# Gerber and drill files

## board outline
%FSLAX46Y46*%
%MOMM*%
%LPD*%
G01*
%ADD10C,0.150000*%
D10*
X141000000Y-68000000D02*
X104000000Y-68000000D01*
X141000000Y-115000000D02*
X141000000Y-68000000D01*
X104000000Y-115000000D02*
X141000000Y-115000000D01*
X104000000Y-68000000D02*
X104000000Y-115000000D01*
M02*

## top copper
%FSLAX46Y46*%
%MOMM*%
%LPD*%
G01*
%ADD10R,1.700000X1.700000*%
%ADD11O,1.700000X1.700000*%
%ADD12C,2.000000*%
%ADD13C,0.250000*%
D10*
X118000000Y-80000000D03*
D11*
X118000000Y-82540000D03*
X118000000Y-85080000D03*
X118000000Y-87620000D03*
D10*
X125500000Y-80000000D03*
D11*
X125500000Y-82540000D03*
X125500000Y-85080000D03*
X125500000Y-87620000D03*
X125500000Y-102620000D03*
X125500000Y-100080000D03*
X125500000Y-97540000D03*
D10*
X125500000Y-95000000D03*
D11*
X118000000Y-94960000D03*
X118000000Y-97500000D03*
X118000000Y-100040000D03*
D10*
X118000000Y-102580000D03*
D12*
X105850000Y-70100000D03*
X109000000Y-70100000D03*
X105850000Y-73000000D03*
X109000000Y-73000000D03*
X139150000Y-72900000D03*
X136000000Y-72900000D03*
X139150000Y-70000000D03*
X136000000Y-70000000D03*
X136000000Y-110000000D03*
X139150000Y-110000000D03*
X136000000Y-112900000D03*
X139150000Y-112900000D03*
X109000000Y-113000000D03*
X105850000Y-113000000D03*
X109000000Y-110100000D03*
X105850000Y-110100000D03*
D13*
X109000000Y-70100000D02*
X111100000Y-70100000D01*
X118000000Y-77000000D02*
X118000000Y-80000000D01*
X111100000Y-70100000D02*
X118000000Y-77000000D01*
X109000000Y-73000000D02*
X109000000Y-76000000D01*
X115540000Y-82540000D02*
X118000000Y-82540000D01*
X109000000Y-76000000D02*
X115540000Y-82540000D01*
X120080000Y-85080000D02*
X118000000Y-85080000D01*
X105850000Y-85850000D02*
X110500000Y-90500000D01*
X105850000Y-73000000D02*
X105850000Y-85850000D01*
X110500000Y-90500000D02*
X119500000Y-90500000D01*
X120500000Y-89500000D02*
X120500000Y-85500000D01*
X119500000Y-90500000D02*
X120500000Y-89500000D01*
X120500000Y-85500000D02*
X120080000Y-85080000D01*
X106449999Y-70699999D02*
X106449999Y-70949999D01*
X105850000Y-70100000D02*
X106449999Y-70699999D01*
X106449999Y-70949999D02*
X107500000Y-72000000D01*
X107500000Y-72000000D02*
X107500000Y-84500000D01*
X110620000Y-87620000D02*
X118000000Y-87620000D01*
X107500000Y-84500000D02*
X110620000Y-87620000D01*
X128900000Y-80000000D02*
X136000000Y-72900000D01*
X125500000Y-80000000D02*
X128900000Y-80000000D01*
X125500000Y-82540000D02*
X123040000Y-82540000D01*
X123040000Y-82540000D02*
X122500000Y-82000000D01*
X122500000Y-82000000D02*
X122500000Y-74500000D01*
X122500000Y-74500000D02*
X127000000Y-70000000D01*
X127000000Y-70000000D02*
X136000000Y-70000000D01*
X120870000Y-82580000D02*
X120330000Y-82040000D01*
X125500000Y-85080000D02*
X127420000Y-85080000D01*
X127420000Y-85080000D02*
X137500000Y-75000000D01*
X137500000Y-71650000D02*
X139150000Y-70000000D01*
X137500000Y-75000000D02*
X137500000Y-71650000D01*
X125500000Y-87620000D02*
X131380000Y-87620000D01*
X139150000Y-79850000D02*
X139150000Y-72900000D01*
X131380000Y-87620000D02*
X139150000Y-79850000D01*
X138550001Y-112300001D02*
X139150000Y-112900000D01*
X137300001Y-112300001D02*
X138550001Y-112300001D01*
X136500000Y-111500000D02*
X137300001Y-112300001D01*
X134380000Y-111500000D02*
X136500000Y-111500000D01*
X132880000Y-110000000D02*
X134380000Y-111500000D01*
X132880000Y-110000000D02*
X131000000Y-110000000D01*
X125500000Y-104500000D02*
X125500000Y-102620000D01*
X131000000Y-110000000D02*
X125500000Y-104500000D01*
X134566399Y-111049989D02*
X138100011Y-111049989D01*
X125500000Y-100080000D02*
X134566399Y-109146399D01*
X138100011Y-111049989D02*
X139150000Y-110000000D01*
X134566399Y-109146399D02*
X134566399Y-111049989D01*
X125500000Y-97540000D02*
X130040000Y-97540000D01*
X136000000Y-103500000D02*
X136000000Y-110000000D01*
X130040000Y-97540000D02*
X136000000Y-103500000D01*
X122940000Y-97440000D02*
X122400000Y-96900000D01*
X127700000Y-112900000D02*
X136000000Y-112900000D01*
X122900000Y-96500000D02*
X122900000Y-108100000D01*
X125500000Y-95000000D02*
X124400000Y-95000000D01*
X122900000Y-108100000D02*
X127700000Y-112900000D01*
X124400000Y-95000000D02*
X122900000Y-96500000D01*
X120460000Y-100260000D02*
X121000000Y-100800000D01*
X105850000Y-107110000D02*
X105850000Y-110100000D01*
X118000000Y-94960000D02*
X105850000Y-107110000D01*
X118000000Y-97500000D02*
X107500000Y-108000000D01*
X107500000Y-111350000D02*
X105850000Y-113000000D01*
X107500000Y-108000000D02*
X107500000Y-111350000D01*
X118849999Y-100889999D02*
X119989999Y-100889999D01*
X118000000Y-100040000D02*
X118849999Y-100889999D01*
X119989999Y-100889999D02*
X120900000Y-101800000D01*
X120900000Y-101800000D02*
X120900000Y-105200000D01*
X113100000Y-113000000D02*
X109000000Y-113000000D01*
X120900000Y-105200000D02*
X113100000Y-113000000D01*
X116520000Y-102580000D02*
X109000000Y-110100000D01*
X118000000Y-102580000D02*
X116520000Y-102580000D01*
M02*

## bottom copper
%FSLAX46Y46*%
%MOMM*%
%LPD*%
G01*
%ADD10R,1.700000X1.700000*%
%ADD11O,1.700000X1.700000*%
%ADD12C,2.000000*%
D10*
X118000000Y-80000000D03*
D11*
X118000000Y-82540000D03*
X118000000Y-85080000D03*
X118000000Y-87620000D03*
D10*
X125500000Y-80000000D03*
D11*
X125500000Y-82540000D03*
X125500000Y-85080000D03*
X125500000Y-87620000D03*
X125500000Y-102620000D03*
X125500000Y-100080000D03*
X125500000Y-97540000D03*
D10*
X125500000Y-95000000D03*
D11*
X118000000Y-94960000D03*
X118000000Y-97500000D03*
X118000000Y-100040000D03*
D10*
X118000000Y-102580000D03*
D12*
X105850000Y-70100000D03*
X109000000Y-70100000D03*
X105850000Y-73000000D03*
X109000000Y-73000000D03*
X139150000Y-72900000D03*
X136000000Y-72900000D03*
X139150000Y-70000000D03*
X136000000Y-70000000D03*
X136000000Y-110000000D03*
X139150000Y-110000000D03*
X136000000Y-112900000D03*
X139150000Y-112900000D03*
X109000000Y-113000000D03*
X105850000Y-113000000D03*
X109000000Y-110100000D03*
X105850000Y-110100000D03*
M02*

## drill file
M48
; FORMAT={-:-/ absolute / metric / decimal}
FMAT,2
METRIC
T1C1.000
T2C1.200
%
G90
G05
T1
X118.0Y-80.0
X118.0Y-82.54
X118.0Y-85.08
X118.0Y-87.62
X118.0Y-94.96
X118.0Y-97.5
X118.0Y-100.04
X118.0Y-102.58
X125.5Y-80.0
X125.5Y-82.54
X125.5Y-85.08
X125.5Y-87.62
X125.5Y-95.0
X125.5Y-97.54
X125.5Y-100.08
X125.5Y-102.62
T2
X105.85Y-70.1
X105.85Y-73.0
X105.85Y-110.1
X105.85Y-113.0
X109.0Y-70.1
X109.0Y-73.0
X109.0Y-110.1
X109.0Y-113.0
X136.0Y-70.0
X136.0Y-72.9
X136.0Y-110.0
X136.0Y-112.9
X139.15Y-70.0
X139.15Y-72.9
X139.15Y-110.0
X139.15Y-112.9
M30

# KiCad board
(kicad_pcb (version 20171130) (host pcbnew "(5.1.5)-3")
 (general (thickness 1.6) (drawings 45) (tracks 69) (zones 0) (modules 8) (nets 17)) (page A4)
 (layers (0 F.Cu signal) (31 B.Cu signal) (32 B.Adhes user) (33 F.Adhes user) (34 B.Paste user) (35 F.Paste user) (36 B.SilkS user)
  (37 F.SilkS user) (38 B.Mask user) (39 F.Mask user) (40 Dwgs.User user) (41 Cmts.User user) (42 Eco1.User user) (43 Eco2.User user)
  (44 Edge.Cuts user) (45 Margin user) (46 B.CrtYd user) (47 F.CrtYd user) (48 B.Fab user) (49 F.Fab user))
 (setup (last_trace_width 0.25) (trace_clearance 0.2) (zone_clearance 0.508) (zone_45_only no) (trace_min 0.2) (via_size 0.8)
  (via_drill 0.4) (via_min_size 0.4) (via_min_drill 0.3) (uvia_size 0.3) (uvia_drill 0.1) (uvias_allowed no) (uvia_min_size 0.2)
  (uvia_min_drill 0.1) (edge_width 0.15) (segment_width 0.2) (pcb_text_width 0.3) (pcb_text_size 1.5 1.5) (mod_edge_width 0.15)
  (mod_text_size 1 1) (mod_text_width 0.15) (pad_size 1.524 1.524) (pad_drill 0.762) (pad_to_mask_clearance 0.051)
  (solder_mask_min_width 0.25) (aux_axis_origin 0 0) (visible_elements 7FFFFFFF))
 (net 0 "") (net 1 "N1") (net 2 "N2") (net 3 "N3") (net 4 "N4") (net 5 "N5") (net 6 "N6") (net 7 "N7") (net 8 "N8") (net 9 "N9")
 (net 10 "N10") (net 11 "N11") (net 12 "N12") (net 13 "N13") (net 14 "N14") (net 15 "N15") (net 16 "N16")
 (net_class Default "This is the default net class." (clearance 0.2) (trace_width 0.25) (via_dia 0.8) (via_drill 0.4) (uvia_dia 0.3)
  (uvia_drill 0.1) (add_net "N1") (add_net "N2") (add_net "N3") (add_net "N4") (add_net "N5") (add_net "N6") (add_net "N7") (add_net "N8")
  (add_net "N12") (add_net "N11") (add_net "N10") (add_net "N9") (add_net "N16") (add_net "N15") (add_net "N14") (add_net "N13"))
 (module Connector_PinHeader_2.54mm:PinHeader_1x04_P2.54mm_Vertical (layer F.Cu) (at 118 80)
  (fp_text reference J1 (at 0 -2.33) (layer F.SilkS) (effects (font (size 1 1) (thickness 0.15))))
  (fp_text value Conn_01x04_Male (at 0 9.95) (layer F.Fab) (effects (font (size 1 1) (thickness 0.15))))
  (pad 1 thru_hole rect (at 0 0) (size 1.7 1.7) (drill 1) (layers *.Cu *.Mask) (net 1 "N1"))
  (pad 2 thru_hole oval (at 0 2.54) (size 1.7 1.7) (drill 1) (layers *.Cu *.Mask) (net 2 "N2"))
  (pad 3 thru_hole oval (at 0 5.08) (size 1.7 1.7) (drill 1) (layers *.Cu *.Mask) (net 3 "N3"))
  (pad 4 thru_hole oval (at 0 7.62) (size 1.7 1.7) (drill 1) (layers *.Cu *.Mask) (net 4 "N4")))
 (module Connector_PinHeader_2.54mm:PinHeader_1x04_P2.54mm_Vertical (layer F.Cu) (at 125.5 80)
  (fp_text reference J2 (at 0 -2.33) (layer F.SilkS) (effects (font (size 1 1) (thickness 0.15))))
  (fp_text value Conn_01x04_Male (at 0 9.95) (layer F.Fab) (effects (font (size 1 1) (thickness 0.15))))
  (pad 1 thru_hole rect (at 0 0) (size 1.7 1.7) (drill 1) (layers *.Cu *.Mask) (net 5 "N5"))
  (pad 2 thru_hole oval (at 0 2.54) (size 1.7 1.7) (drill 1) (layers *.Cu *.Mask) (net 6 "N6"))
  (pad 3 thru_hole oval (at 0 5.08) (size 1.7 1.7) (drill 1) (layers *.Cu *.Mask) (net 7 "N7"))
  (pad 4 thru_hole oval (at 0 7.62) (size 1.7 1.7) (drill 1) (layers *.Cu *.Mask) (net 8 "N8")))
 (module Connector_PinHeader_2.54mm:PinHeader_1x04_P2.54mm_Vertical (layer F.Cu) (at 125.5 95)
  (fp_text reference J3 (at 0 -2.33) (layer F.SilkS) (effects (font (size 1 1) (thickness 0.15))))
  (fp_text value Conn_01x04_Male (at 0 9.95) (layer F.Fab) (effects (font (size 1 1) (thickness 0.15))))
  (pad 4 thru_hole oval (at 0 7.62) (size 1.7 1.7) (drill 1) (layers *.Cu *.Mask) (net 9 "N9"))
  (pad 3 thru_hole oval (at 0 5.08) (size 1.7 1.7) (drill 1) (layers *.Cu *.Mask) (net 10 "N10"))
  (pad 2 thru_hole oval (at 0 2.54) (size 1.7 1.7) (drill 1) (layers *.Cu *.Mask) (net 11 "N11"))
  (pad 1 thru_hole rect (at 0 0) (size 1.7 1.7) (drill 1) (layers *.Cu *.Mask) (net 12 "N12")))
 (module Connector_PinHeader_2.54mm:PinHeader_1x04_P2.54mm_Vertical (layer F.Cu) (at 118 102.58 180)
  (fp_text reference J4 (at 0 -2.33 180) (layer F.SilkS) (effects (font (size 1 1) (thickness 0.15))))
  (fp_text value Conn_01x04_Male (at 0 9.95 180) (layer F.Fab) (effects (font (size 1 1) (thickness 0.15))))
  (pad 4 thru_hole oval (at 0 7.62 180) (size 1.7 1.7) (drill 1) (layers *.Cu *.Mask) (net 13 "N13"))
  (pad 3 thru_hole oval (at 0 5.08 180) (size 1.7 1.7) (drill 1) (layers *.Cu *.Mask) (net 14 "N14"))
  (pad 2 thru_hole oval (at 0 2.54 180) (size 1.7 1.7) (drill 1) (layers *.Cu *.Mask) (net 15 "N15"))
  (pad 1 thru_hole rect (at 0 0 180) (size 1.7 1.7) (drill 1) (layers *.Cu *.Mask) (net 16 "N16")))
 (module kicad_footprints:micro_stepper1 (layer F.Cu) (at 107.5 71.5 180)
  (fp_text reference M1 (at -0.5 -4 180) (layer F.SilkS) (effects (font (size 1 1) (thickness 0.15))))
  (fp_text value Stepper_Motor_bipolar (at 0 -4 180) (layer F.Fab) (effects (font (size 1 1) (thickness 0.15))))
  (pad 4 thru_hole circle (at 1.65 1.4 180) (size 2 2) (drill 1.2) (layers *.Cu *.Mask) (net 4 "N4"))
  (pad 2 thru_hole circle (at -1.5 1.4 180) (size 2 2) (drill 1.2) (layers *.Cu *.Mask) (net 1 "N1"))
  (pad 3 thru_hole circle (at 1.65 -1.5 180) (size 2 2) (drill 1.2) (layers *.Cu *.Mask) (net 3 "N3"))
  (pad 1 thru_hole circle (at -1.5 -1.5 180) (size 2 2) (drill 1.2) (layers *.Cu *.Mask) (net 2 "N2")))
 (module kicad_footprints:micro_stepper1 (layer F.Cu) (at 137.5 71.5)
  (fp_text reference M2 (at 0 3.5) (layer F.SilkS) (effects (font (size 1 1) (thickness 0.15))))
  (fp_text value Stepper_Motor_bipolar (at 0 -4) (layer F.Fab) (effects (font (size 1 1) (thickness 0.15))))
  (pad 4 thru_hole circle (at 1.65 1.4) (size 2 2) (drill 1.2) (layers *.Cu *.Mask) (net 8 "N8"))
  (pad 2 thru_hole circle (at -1.5 1.4) (size 2 2) (drill 1.2) (layers *.Cu *.Mask) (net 5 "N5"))
  (pad 3 thru_hole circle (at 1.65 -1.5) (size 2 2) (drill 1.2) (layers *.Cu *.Mask) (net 7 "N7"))
  (pad 1 thru_hole circle (at -1.5 -1.5) (size 2 2) (drill 1.2) (layers *.Cu *.Mask) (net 6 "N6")))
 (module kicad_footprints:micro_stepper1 (layer F.Cu) (at 137.5 111.5)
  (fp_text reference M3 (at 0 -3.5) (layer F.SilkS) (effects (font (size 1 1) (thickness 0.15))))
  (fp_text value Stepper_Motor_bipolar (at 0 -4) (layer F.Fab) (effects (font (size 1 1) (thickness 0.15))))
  (pad 1 thru_hole circle (at -1.5 -1.5) (size 2 2) (drill 1.2) (layers *.Cu *.Mask) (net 11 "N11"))
  (pad 3 thru_hole circle (at 1.65 -1.5) (size 2 2) (drill 1.2) (layers *.Cu *.Mask) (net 10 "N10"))
  (pad 2 thru_hole circle (at -1.5 1.4) (size 2 2) (drill 1.2) (layers *.Cu *.Mask) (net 12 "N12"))
  (pad 4 thru_hole circle (at 1.65 1.4) (size 2 2) (drill 1.2) (layers *.Cu *.Mask) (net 9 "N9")))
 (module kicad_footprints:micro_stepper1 (layer F.Cu) (at 107.5 111.5 180)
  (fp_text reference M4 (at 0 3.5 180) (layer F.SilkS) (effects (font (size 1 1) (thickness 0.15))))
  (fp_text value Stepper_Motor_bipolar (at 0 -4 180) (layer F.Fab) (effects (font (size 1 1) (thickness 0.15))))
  (pad 1 thru_hole circle (at -1.5 -1.5 180) (size 2 2) (drill 1.2) (layers *.Cu *.Mask) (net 15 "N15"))
  (pad 3 thru_hole circle (at 1.65 -1.5 180) (size 2 2) (drill 1.2) (layers *.Cu *.Mask) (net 14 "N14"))
  (pad 2 thru_hole circle (at -1.5 1.4 180) (size 2 2) (drill 1.2) (layers *.Cu *.Mask) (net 16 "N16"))
  (pad 4 thru_hole circle (at 1.65 1.4 180) (size 2 2) (drill 1.2) (layers *.Cu *.Mask) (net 13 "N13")))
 (gr_line (start 141 68) (end 104 68) (layer Edge.Cuts) (width 0.15))
 (gr_line (start 141 115) (end 141 68) (layer Edge.Cuts) (width 0.15))
 (gr_line (start 104 115) (end 141 115) (layer Edge.Cuts) (width 0.15))
 (gr_line (start 104 68) (end 104 115) (layer Edge.Cuts) (width 0.15))
 (segment (start 109 70.1) (end 111.1 70.1) (width 0.25) (layer F.Cu) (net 1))
 (segment (start 118 77) (end 118 80) (width 0.25) (layer F.Cu) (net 1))
 (segment (start 111.1 70.1) (end 118 77) (width 0.25) (layer F.Cu) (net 1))
 (segment (start 109 73) (end 109 76) (width 0.25) (layer F.Cu) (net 2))
 (segment (start 115.54 82.54) (end 118 82.54) (width 0.25) (layer F.Cu) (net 2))
 (segment (start 109 76) (end 115.54 82.54) (width 0.25) (layer F.Cu) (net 2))
 (segment (start 120.08 85.08) (end 118 85.08) (width 0.25) (layer F.Cu) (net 3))
 (segment (start 105.85 85.85) (end 110.5 90.5) (width 0.25) (layer F.Cu) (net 3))
 (segment (start 105.85 73) (end 105.85 85.85) (width 0.25) (layer F.Cu) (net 3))
 (segment (start 110.5 90.5) (end 119.5 90.5) (width 0.25) (layer F.Cu) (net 3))
 (segment (start 120.5 89.5) (end 120.5 85.5) (width 0.25) (layer F.Cu) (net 3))
 (segment (start 119.5 90.5) (end 120.5 89.5) (width 0.25) (layer F.Cu) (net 3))
 (segment (start 120.5 85.5) (end 120.08 85.08) (width 0.25) (layer F.Cu) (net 3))
 (segment (start 106.449999 70.699999) (end 106.449999 70.949999) (width 0.25) (layer F.Cu) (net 4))
 (segment (start 105.85 70.1) (end 106.449999 70.699999) (width 0.25) (layer F.Cu) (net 4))
 (segment (start 106.449999 70.949999) (end 107.5 72) (width 0.25) (layer F.Cu) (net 4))
 (segment (start 107.5 72) (end 107.5 84.5) (width 0.25) (layer F.Cu) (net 4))
 (segment (start 110.62 87.62) (end 118 87.62) (width 0.25) (layer F.Cu) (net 4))
 (segment (start 107.5 84.5) (end 110.62 87.62) (width 0.25) (layer F.Cu) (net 4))
 (segment (start 128.9 80) (end 136 72.9) (width 0.25) (layer F.Cu) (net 5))
 (segment (start 125.5 80) (end 128.9 80) (width 0.25) (layer F.Cu) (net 5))
 (segment (start 125.5 82.54) (end 123.04 82.54) (width 0.25) (layer F.Cu) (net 6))
 (segment (start 123.04 82.54) (end 122.5 82) (width 0.25) (layer F.Cu) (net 6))
 (segment (start 122.5 82) (end 122.5 74.5) (width 0.25) (layer F.Cu) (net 6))
 (segment (start 122.5 74.5) (end 127 70) (width 0.25) (layer F.Cu) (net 6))
 (segment (start 127 70) (end 136 70) (width 0.25) (layer F.Cu) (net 6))
 (segment (start 120.87 82.58) (end 120.33 82.04) (width 0.25) (layer F.Cu) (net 6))
 (segment (start 125.5 85.08) (end 127.42 85.08) (width 0.25) (layer F.Cu) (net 7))
 (segment (start 127.42 85.08) (end 137.5 75) (width 0.25) (layer F.Cu) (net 7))
 (segment (start 137.5 71.65) (end 139.15 70) (width 0.25) (layer F.Cu) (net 7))
 (segment (start 137.5 75) (end 137.5 71.65) (width 0.25) (layer F.Cu) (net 7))
 (segment (start 125.5 87.62) (end 131.38 87.62) (width 0.25) (layer F.Cu) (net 8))
 (segment (start 139.15 79.85) (end 139.15 72.9) (width 0.25) (layer F.Cu) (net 8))
 (segment (start 131.38 87.62) (end 139.15 79.85) (width 0.25) (layer F.Cu) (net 8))
 (segment (start 138.550001 112.300001) (end 139.15 112.9) (width 0.25) (layer F.Cu) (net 9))
 (segment (start 137.300001 112.300001) (end 138.550001 112.300001) (width 0.25) (layer F.Cu) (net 9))
 (segment (start 136.5 111.5) (end 137.300001 112.300001) (width 0.25) (layer F.Cu) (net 9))
 (segment (start 134.38 111.5) (end 136.5 111.5) (width 0.25) (layer F.Cu) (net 9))
 (segment (start 132.88 110) (end 134.38 111.5) (width 0.25) (layer F.Cu) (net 9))
 (segment (start 132.88 110) (end 131 110) (width 0.25) (layer F.Cu) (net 9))
 (segment (start 125.5 104.5) (end 125.5 102.62) (width 0.25) (layer F.Cu) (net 9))
 (segment (start 131 110) (end 125.5 104.5) (width 0.25) (layer F.Cu) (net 9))
 (segment (start 134.566399 111.049989) (end 138.100011 111.049989) (width 0.25) (layer F.Cu) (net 10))
 (segment (start 125.5 100.08) (end 134.566399 109.146399) (width 0.25) (layer F.Cu) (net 10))
 (segment (start 138.100011 111.049989) (end 139.15 110) (width 0.25) (layer F.Cu) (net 10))
 (segment (start 134.566399 109.146399) (end 134.566399 111.049989) (width 0.25) (layer F.Cu) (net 10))
 (segment (start 125.5 97.54) (end 130.04 97.54) (width 0.25) (layer F.Cu) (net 11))
 (segment (start 136 103.5) (end 136 110) (width 0.25) (layer F.Cu) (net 11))
 (segment (start 130.04 97.54) (end 136 103.5) (width 0.25) (layer F.Cu) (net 11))
 (segment (start 122.94 97.44) (end 122.4 96.9) (width 0.25) (layer F.Cu) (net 12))
 (segment (start 127.7 112.9) (end 136 112.9) (width 0.25) (layer F.Cu) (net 12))
 (segment (start 122.9 96.5) (end 122.9 108.1) (width 0.25) (layer F.Cu) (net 12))
 (segment (start 125.5 95) (end 124.4 95) (width 0.25) (layer F.Cu) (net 12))
 (segment (start 122.9 108.1) (end 127.7 112.9) (width 0.25) (layer F.Cu) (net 12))
 (segment (start 124.4 95) (end 122.9 96.5) (width 0.25) (layer F.Cu) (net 12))
 (segment (start 120.46 100.26) (end 121 100.8) (width 0.25) (layer F.Cu) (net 12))
 (segment (start 105.85 107.11) (end 105.85 110.1) (width 0.25) (layer F.Cu) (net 13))
 (segment (start 118 94.96) (end 105.85 107.11) (width 0.25) (layer F.Cu) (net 13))
 (segment (start 118 97.5) (end 107.5 108) (width 0.25) (layer F.Cu) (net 14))
 (segment (start 107.5 111.35) (end 105.85 113) (width 0.25) (layer F.Cu) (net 14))
 (segment (start 107.5 108) (end 107.5 111.35) (width 0.25) (layer F.Cu) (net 14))
 (segment (start 118.849999 100.889999) (end 119.989999 100.889999) (width 0.25) (layer F.Cu) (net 15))
 (segment (start 118 100.04) (end 118.849999 100.889999) (width 0.25) (layer F.Cu) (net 15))
 (segment (start 119.989999 100.889999) (end 120.9 101.8) (width 0.25) (layer F.Cu) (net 15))
 (segment (start 120.9 101.8) (end 120.9 105.2) (width 0.25) (layer F.Cu) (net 15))
 (segment (start 113.1 113) (end 109 113) (width 0.25) (layer F.Cu) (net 15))
 (segment (start 120.9 105.2) (end 113.1 113) (width 0.25) (layer F.Cu) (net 15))
 (segment (start 116.52 102.58) (end 109 110.1) (width 0.25) (layer F.Cu) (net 16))
 (segment (start 118 102.58) (end 116.52 102.58) (width 0.25) (layer F.Cu) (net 16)))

